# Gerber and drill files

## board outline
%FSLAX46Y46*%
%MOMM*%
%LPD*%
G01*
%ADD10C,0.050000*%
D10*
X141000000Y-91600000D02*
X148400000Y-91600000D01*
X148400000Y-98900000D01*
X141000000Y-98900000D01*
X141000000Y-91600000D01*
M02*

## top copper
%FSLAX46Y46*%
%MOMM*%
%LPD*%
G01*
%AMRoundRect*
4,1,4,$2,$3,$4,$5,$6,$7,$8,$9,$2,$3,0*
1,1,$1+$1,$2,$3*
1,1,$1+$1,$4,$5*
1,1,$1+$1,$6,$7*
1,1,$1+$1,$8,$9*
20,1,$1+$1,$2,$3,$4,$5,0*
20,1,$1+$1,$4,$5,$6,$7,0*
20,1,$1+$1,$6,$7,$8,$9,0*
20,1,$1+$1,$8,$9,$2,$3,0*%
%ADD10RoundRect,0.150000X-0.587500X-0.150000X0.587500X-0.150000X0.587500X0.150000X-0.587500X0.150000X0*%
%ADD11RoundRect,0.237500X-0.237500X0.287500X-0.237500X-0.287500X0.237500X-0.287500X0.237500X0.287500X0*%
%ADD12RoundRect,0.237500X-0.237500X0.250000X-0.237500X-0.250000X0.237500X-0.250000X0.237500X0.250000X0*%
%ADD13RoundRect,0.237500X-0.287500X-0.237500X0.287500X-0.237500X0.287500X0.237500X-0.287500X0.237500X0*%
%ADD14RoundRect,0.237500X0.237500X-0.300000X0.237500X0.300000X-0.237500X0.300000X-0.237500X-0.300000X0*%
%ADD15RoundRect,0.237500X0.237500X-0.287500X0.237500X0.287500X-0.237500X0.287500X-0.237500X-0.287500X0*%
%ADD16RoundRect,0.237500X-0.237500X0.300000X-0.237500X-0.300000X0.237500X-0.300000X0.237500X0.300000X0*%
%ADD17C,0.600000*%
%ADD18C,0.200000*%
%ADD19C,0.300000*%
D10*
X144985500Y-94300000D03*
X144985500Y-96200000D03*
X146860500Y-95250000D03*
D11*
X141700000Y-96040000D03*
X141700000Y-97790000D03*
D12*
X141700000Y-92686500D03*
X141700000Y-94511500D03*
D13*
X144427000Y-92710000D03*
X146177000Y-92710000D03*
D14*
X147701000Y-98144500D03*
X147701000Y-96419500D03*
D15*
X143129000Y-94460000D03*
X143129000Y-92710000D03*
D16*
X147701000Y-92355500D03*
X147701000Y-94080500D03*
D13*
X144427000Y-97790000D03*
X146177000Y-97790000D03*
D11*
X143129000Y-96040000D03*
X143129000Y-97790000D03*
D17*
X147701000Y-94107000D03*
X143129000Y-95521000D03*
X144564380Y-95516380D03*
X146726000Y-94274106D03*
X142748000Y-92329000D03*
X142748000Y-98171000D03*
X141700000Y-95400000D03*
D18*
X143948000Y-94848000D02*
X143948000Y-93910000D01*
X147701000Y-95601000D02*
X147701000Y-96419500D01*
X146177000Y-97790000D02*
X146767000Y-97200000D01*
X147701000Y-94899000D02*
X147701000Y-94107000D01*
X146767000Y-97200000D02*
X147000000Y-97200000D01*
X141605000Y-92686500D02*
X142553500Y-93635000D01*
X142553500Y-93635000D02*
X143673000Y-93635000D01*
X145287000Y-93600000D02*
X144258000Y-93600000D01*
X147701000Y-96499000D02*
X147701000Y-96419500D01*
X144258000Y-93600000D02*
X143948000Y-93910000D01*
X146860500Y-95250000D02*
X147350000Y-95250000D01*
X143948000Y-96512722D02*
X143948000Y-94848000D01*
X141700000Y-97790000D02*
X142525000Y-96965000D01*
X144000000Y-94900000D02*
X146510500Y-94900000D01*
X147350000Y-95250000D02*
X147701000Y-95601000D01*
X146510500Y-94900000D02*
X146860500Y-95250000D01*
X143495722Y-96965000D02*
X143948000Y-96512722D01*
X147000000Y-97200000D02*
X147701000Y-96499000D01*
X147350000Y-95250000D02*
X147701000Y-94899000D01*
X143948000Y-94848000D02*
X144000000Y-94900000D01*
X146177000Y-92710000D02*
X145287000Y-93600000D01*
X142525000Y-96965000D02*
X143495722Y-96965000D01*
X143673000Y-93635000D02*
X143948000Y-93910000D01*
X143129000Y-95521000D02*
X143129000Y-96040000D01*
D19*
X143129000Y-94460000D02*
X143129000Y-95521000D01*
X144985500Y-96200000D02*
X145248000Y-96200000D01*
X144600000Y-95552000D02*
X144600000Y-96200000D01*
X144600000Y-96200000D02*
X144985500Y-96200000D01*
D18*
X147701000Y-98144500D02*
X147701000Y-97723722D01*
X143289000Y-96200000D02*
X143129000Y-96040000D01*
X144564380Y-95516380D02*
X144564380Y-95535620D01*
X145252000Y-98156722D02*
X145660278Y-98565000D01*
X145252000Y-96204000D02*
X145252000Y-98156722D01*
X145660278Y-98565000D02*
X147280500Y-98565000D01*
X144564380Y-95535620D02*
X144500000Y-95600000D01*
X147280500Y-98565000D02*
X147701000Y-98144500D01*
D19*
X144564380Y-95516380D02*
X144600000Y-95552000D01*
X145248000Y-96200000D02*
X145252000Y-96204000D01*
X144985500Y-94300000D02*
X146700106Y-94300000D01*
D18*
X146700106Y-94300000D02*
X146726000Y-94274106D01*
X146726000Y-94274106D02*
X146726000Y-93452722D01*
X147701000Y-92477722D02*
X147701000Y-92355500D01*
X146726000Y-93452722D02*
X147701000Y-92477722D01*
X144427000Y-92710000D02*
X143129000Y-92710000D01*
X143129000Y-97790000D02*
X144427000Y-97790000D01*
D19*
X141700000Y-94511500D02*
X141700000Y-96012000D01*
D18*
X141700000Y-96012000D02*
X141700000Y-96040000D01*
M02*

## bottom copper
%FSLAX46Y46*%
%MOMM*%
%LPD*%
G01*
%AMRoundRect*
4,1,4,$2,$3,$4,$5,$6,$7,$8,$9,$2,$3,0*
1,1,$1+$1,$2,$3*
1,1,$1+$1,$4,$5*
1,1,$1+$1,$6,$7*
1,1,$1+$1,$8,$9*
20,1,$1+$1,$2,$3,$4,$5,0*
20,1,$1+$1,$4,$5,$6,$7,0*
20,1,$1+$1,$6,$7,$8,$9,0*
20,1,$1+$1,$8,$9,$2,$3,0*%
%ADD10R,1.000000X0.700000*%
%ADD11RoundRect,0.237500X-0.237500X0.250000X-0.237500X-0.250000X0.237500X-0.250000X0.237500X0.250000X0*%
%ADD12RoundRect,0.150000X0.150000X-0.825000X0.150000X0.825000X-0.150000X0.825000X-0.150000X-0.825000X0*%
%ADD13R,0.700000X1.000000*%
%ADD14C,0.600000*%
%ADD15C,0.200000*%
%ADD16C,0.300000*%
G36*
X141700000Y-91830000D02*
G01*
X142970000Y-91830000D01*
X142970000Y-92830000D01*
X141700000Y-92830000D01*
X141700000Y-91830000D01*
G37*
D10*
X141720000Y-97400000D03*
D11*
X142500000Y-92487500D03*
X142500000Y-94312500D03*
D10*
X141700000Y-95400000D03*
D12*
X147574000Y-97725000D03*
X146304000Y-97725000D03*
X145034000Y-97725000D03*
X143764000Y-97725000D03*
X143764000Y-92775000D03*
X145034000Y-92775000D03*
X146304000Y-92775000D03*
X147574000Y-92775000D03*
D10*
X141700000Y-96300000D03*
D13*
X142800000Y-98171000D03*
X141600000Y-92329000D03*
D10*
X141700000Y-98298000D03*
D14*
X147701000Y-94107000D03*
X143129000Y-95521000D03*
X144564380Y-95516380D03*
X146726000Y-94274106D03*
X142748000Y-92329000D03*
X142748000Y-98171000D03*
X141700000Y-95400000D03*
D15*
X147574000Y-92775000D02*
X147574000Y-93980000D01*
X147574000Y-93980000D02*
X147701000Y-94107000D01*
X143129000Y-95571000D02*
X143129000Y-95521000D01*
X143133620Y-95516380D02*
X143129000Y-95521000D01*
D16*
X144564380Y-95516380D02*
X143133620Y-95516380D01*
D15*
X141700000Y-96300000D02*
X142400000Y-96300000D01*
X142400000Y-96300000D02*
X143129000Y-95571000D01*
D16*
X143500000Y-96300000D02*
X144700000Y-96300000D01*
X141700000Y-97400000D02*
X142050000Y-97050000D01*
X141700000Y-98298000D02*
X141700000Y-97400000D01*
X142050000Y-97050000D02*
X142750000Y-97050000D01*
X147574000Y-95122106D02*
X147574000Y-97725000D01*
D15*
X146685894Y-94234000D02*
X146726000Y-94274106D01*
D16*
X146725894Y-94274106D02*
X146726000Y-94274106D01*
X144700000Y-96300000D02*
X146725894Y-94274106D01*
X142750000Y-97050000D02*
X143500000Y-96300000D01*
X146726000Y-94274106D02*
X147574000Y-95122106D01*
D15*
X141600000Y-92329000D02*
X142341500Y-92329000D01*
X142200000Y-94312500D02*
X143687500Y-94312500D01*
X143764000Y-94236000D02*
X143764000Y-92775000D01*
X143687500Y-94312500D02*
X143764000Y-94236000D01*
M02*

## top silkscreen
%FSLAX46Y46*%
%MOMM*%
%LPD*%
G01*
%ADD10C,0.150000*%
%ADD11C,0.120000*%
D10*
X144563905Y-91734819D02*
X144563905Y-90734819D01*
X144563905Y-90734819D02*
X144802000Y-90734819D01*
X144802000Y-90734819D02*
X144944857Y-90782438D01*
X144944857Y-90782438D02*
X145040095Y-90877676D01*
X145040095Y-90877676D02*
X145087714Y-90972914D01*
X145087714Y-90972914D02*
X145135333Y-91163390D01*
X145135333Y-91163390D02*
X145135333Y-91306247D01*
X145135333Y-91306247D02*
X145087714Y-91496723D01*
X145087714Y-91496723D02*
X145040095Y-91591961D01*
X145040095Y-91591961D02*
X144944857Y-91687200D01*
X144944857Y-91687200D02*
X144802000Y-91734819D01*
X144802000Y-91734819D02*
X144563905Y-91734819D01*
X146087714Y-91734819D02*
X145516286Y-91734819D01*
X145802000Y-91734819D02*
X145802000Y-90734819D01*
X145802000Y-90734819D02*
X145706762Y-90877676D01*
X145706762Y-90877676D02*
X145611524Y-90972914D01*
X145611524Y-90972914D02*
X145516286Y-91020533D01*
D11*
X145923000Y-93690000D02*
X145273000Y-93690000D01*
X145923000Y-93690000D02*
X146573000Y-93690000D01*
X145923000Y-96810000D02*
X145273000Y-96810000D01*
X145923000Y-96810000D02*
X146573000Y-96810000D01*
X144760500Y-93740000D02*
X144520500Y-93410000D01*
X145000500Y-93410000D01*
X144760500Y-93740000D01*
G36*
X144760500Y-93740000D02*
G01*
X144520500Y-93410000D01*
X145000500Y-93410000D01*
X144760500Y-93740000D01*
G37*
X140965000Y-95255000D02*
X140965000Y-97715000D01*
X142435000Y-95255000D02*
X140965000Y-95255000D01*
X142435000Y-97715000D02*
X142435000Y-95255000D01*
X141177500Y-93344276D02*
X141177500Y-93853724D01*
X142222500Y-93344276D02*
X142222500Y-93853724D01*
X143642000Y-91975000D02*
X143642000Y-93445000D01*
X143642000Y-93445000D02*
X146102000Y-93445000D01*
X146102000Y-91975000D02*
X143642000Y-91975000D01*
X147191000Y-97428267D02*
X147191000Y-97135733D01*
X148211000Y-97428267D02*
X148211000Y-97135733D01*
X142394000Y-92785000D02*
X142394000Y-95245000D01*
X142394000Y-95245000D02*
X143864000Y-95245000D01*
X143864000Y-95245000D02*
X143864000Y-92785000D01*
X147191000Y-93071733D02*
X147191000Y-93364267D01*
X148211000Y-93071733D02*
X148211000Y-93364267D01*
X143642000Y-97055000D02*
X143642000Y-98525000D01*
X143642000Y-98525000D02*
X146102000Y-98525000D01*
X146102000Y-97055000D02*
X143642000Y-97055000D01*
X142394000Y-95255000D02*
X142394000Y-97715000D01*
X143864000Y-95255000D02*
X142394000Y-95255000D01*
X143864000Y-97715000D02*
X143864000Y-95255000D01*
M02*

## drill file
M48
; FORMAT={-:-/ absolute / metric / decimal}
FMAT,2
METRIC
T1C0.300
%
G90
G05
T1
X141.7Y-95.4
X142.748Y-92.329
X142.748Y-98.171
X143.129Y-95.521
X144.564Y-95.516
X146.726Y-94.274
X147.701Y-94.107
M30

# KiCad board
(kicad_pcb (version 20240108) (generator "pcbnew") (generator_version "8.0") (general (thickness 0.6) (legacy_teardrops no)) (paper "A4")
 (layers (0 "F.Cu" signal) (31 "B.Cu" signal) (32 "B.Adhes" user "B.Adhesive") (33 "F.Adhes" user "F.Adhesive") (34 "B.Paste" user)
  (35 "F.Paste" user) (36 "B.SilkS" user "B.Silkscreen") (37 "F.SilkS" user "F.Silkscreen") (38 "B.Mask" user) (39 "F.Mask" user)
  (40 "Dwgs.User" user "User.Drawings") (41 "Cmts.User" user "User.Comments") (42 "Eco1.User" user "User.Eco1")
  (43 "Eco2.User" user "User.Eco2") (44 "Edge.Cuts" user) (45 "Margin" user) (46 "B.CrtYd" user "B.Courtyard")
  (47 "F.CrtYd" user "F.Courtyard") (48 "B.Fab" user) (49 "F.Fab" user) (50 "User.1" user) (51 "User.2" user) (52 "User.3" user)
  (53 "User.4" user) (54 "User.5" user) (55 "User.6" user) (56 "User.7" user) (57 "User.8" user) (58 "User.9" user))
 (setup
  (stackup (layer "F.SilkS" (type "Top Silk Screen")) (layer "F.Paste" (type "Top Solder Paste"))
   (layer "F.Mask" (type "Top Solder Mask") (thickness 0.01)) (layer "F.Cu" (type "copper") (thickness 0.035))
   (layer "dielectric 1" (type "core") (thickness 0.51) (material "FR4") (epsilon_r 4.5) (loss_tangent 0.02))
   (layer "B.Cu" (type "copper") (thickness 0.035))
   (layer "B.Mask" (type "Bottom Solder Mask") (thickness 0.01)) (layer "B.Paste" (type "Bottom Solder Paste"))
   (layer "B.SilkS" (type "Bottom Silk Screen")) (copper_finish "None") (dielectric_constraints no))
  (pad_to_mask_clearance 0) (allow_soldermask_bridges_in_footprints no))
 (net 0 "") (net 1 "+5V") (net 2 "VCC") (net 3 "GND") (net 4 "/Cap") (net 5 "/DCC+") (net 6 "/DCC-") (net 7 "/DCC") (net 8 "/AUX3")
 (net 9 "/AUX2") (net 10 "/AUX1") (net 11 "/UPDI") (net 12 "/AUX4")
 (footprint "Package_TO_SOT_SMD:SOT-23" (layer "F.Cu") (at 145.923 95.25)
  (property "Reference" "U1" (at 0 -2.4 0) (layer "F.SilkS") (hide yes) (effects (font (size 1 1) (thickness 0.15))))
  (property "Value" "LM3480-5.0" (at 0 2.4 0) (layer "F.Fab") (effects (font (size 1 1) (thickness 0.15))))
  (fp_line (start 0 -1.56) (end -0.65 -1.56) (stroke (width 0.12) (type solid)) (layer "F.SilkS"))
  (fp_line (start 0 -1.56) (end 0.65 -1.56) (stroke (width 0.12) (type solid)) (layer "F.SilkS"))
  (fp_line (start 0 1.56) (end -0.65 1.56) (stroke (width 0.12) (type solid)) (layer "F.SilkS"))
  (fp_line (start 0 1.56) (end 0.65 1.56) (stroke (width 0.12) (type solid)) (layer "F.SilkS"))
  (fp_poly
   (pts (xy -1.1625 -1.51) (xy -1.4025 -1.84) (xy -0.9225 -1.84) (xy -1.1625 -1.51)) (stroke (width 0.12) (type solid)) (fill solid)
   (layer "F.SilkS"))
  (pad "1" smd roundrect (at -0.9375 -0.95) (size 1.475 0.6) (layers "F.Cu" "F.Paste" "F.Mask") (roundrect_rratio 0.25) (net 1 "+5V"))
  (pad "2" smd roundrect (at -0.9375 0.95) (size 1.475 0.6) (layers "F.Cu" "F.Paste" "F.Mask") (roundrect_rratio 0.25) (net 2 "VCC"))
  (pad "3" smd roundrect (at 0.9375 0) (size 1.475 0.6) (layers "F.Cu" "F.Paste" "F.Mask") (roundrect_rratio 0.25) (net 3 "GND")))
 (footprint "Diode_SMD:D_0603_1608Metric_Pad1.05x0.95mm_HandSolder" (layer "F.Cu") (at 141.7 96.915 -90)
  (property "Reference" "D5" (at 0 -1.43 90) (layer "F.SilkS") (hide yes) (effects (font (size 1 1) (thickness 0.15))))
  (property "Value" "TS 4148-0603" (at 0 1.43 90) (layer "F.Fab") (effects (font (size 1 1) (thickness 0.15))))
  (fp_line (start -1.66 0.735) (end 0.8 0.735) (stroke (width 0.12) (type solid)) (layer "F.SilkS"))
  (fp_line (start -1.66 -0.735) (end -1.66 0.735) (stroke (width 0.12) (type solid)) (layer "F.SilkS"))
  (fp_line (start 0.8 -0.735) (end -1.66 -0.735) (stroke (width 0.12) (type solid)) (layer "F.SilkS"))
  (pad "1" smd roundrect (at -0.875 0 270) (size 1.05 0.95) (layers "F.Cu" "F.Paste" "F.Mask") (roundrect_rratio 0.25) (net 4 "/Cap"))
  (pad "2" smd roundrect (at 0.875 0 270) (size 1.05 0.95) (layers "F.Cu" "F.Paste" "F.Mask") (roundrect_rratio 0.25) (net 3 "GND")))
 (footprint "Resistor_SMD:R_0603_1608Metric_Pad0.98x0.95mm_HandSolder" (layer "F.Cu") (at 141.7 93.599 -90)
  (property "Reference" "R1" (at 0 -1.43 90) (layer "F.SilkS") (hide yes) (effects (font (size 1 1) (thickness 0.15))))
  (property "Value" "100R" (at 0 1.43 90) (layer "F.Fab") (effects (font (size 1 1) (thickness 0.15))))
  (fp_line (start -0.254724 0.5225) (end 0.254724 0.5225) (stroke (width 0.12) (type solid)) (layer "F.SilkS"))
  (fp_line (start -0.254724 -0.5225) (end 0.254724 -0.5225) (stroke (width 0.12) (type solid)) (layer "F.SilkS"))
  (pad "1" smd roundrect (at -0.9125 0 270) (size 0.975 0.95) (layers "F.Cu" "F.Paste" "F.Mask") (roundrect_rratio 0.25) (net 3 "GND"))
  (pad "2" smd roundrect (at 0.9125 0 270) (size 0.975 0.95) (layers "F.Cu" "F.Paste" "F.Mask") (roundrect_rratio 0.25) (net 4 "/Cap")))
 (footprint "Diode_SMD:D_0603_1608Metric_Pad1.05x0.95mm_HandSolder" (layer "F.Cu") (at 145.302 92.71)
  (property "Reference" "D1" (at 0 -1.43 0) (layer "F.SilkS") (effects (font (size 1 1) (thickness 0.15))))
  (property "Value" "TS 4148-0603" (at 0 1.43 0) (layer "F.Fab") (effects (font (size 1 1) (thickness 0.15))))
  (fp_line (start -1.66 -0.735) (end -1.66 0.735) (stroke (width 0.12) (type solid)) (layer "F.SilkS"))
  (fp_line (start -1.66 0.735) (end 0.8 0.735) (stroke (width 0.12) (type solid)) (layer "F.SilkS"))
  (fp_line (start 0.8 -0.735) (end -1.66 -0.735) (stroke (width 0.12) (type solid)) (layer "F.SilkS"))
  (pad "1" smd roundrect (at -0.875 0) (size 1.05 0.95) (layers "F.Cu" "F.Paste" "F.Mask") (roundrect_rratio 0.25) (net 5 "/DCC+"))
  (pad "2" smd roundrect (at 0.875 0) (size 1.05 0.95) (layers "F.Cu" "F.Paste" "F.Mask") (roundrect_rratio 0.25) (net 3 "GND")))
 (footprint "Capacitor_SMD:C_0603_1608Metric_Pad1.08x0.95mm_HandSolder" (layer "F.Cu") (at 147.701 97.282 90)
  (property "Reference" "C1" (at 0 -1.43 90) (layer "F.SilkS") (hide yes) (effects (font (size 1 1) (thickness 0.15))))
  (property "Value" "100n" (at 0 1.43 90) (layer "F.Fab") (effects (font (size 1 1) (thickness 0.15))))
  (fp_line (start -0.146267 -0.51) (end 0.146267 -0.51) (stroke (width 0.12) (type solid)) (layer "F.SilkS"))
  (fp_line (start -0.146267 0.51) (end 0.146267 0.51) (stroke (width 0.12) (type solid)) (layer "F.SilkS"))
  (pad "1" smd roundrect (at -0.8625 0 90) (size 1.075 0.95) (layers "F.Cu" "F.Paste" "F.Mask") (roundrect_rratio 0.25) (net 2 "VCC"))
  (pad "2" smd roundrect (at 0.8625 0 90) (size 1.075 0.95) (layers "F.Cu" "F.Paste" "F.Mask") (roundrect_rratio 0.25) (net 3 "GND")))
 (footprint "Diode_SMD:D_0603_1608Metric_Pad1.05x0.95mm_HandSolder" (layer "F.Cu") (at 143.129 93.585 90)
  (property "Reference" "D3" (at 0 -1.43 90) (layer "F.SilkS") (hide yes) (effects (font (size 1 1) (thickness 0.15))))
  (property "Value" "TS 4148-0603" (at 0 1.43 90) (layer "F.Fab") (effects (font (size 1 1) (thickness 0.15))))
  (fp_line (start 0.8 -0.735) (end -1.66 -0.735) (stroke (width 0.12) (type solid)) (layer "F.SilkS"))
  (fp_line (start -1.66 -0.735) (end -1.66 0.735) (stroke (width 0.12) (type solid)) (layer "F.SilkS"))
  (fp_line (start -1.66 0.735) (end 0.8 0.735) (stroke (width 0.12) (type solid)) (layer "F.SilkS"))
  (pad "1" smd roundrect (at -0.875 0 90) (size 1.05 0.95) (layers "F.Cu" "F.Paste" "F.Mask") (roundrect_rratio 0.25) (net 2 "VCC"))
  (pad "2" smd roundrect (at 0.875 0 90) (size 1.05 0.95) (layers "F.Cu" "F.Paste" "F.Mask") (roundrect_rratio 0.25) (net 5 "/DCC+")))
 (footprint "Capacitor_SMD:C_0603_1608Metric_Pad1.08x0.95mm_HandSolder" (layer "F.Cu") (at 147.701 93.218 -90)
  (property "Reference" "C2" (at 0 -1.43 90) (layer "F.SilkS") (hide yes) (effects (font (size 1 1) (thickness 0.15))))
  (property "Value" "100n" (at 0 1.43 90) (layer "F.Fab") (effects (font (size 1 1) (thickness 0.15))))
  (fp_line (start -0.146267 0.51) (end 0.146267 0.51) (stroke (width 0.12) (type solid)) (layer "F.SilkS"))
  (fp_line (start -0.146267 -0.51) (end 0.146267 -0.51) (stroke (width 0.12) (type solid)) (layer "F.SilkS"))
  (pad "1" smd roundrect (at -0.8625 0 270) (size 1.075 0.95) (layers "F.Cu" "F.Paste" "F.Mask") (roundrect_rratio 0.25) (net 1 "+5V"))
  (pad "2" smd roundrect (at 0.8625 0 270) (size 1.075 0.95) (layers "F.Cu" "F.Paste" "F.Mask") (roundrect_rratio 0.25) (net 3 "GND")))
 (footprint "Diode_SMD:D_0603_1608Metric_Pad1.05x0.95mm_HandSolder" (layer "F.Cu") (at 145.302 97.79)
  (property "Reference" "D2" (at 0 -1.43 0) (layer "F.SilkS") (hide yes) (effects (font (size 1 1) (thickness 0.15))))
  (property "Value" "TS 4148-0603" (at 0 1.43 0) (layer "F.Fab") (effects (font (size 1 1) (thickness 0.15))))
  (fp_line (start -1.66 -0.735) (end -1.66 0.735) (stroke (width 0.12) (type solid)) (layer "F.SilkS"))
  (fp_line (start -1.66 0.735) (end 0.8 0.735) (stroke (width 0.12) (type solid)) (layer "F.SilkS"))
  (fp_line (start 0.8 -0.735) (end -1.66 -0.735) (stroke (width 0.12) (type solid)) (layer "F.SilkS"))
  (pad "1" smd roundrect (at -0.875 0) (size 1.05 0.95) (layers "F.Cu" "F.Paste" "F.Mask") (roundrect_rratio 0.25) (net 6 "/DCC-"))
  (pad "2" smd roundrect (at 0.875 0) (size 1.05 0.95) (layers "F.Cu" "F.Paste" "F.Mask") (roundrect_rratio 0.25) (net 3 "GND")))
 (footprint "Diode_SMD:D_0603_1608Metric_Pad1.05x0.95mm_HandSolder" (layer "F.Cu") (at 143.129 96.915 -90)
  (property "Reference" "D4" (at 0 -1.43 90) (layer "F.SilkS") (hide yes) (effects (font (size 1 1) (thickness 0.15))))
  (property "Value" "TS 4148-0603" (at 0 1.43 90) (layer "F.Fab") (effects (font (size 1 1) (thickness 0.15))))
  (fp_line (start -1.66 0.735) (end 0.8 0.735) (stroke (width 0.12) (type solid)) (layer "F.SilkS"))
  (fp_line (start -1.66 -0.735) (end -1.66 0.735) (stroke (width 0.12) (type solid)) (layer "F.SilkS"))
  (fp_line (start 0.8 -0.735) (end -1.66 -0.735) (stroke (width 0.12) (type solid)) (layer "F.SilkS"))
  (pad "1" smd roundrect (at -0.875 0 270) (size 1.05 0.95) (layers "F.Cu" "F.Paste" "F.Mask") (roundrect_rratio 0.25) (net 2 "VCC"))
  (pad "2" smd roundrect (at 0.875 0 270) (size 1.05 0.95) (layers "F.Cu" "F.Paste" "F.Mask") (roundrect_rratio 0.25) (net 6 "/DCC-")))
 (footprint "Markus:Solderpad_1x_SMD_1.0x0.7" (layer "B.Cu") (at 141.72 97.4 180)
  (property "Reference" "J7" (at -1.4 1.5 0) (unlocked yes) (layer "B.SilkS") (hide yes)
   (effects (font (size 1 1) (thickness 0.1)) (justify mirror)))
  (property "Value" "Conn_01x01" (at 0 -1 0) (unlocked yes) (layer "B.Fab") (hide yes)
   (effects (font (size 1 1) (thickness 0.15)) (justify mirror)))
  (pad "1" smd rect (at 0 0 180) (size 1 0.7) (layers "B.Cu" "B.Paste" "B.Mask") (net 1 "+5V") (thermal_bridge_angle 45)))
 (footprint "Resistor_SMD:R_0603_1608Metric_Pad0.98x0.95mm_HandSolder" (layer "B.Cu") (at 142.5 93.4 -90)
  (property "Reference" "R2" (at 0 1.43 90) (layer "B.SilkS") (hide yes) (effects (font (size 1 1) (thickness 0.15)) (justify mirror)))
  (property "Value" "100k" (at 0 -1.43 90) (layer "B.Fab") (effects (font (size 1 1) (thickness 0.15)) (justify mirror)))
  (pad "1" smd roundrect (at -0.9125 0 270) (size 0.975 0.95) (layers "B.Cu" "B.Paste" "B.Mask") (roundrect_rratio 0.25) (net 5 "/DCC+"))
  (pad "2" smd roundrect (at 0.9125 0 270) (size 0.975 0.95) (layers "B.Cu" "B.Paste" "B.Mask") (roundrect_rratio 0.25) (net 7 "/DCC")))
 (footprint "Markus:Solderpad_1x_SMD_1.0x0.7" (layer "B.Cu") (at 141.7 95.4 180)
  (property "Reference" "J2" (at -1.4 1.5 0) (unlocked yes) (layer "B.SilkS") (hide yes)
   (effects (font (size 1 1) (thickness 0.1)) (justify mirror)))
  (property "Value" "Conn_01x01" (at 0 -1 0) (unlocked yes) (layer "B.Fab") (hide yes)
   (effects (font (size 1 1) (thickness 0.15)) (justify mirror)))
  (pad "1" smd rect (at 0 0 180) (size 1 0.7) (layers "B.Cu" "B.Paste" "B.Mask") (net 4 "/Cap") (thermal_bridge_angle 45)))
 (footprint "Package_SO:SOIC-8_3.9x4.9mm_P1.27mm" (layer "B.Cu") (at 145.669 95.25 90)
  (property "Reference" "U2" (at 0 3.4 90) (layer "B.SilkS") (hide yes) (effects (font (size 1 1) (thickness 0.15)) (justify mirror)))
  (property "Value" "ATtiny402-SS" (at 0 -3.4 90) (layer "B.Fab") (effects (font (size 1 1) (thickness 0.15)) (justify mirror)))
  (pad "1" smd roundrect (at -2.475 1.905 90) (size 1.95 0.6) (layers "B.Cu" "B.Paste" "B.Mask") (roundrect_rratio 0.25) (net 1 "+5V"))
  (pad "2" smd roundrect (at -2.475 0.635 90) (size 1.95 0.6) (layers "B.Cu" "B.Paste" "B.Mask") (roundrect_rratio 0.25) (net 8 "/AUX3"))
  (pad "3" smd roundrect (at -2.475 -0.635 90) (size 1.95 0.6) (layers "B.Cu" "B.Paste" "B.Mask") (roundrect_rratio 0.25) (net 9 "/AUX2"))
  (pad "4" smd roundrect (at -2.475 -1.905 90) (size 1.95 0.6) (layers "B.Cu" "B.Paste" "B.Mask") (roundrect_rratio 0.25) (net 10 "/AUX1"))
  (pad "5" smd roundrect (at 2.475 -1.905 90) (size 1.95 0.6) (layers "B.Cu" "B.Paste" "B.Mask") (roundrect_rratio 0.25) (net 7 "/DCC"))
  (pad "6" smd roundrect (at 2.475 -0.635 90) (size 1.95 0.6) (layers "B.Cu" "B.Paste" "B.Mask") (roundrect_rratio 0.25) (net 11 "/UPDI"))
  (pad "7" smd roundrect (at 2.475 0.635 90) (size 1.95 0.6) (layers "B.Cu" "B.Paste" "B.Mask") (roundrect_rratio 0.25) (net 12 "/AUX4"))
  (pad "8" smd roundrect (at 2.475 1.905 90) (size 1.95 0.6) (layers "B.Cu" "B.Paste" "B.Mask") (roundrect_rratio 0.25) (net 3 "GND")))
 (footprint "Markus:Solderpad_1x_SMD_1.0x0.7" (layer "B.Cu") (at 141.7 96.3 180)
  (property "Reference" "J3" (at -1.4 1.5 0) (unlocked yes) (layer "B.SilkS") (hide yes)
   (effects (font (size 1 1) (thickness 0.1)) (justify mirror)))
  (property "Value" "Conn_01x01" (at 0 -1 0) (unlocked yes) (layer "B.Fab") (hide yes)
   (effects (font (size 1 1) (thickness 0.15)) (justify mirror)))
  (pad "1" smd rect (at 0 0 180) (size 1 0.7) (layers "B.Cu" "B.Paste" "B.Mask") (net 2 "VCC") (thermal_bridge_angle 45)))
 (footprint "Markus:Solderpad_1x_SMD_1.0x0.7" (layer "B.Cu") (at 142.8 98.171 -90)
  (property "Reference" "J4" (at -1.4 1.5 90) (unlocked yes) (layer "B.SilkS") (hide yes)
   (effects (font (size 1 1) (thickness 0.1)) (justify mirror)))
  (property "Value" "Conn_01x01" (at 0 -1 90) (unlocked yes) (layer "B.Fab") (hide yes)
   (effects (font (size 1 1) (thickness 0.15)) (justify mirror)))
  (pad "1" smd rect (at 0 0 270) (size 1 0.7) (layers "B.Cu" "B.Paste" "B.Mask") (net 6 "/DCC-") (thermal_bridge_angle 45)))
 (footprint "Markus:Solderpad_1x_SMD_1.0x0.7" (layer "B.Cu") (at 141.6 92.329 -90)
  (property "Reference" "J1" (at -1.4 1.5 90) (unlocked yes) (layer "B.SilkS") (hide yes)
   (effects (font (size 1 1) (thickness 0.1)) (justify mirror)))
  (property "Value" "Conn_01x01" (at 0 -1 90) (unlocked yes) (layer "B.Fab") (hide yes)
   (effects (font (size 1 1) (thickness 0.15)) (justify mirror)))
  (pad "1" smd rect (at 0 0 270) (size 1 0.7) (layers "B.Cu" "B.Paste" "B.Mask") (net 5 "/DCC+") (thermal_bridge_angle 45)))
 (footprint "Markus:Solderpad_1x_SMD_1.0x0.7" (layer "B.Cu") (at 141.7 98.298 180)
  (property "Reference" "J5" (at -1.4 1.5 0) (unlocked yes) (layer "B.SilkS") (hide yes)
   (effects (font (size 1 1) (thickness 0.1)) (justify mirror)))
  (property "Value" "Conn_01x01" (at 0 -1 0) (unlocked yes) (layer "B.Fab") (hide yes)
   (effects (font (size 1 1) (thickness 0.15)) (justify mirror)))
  (pad "1" smd rect (at 0 0 180) (size 1 0.7) (layers "B.Cu" "B.Paste" "B.Mask") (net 1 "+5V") (thermal_bridge_angle 45)))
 (gr_rect (start 141.7 91.83) (end 142.97 92.83) (stroke (width 0) (type solid)) (fill solid) (layer "B.Cu") (net 5))
 (gr_rect (start 141 91.6) (end 148.4 98.9) (stroke (width 0.05) (type default)) (fill none) (layer "Edge.Cuts"))
 (segment (start 143.948 94.848) (end 143.948 93.91) (width 0.2) (layer "F.Cu") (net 3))
 (segment (start 147.701 95.601) (end 147.701 96.4195) (width 0.2) (layer "F.Cu") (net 3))
 (segment (start 146.177 97.79) (end 146.767 97.2) (width 0.2) (layer "F.Cu") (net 3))
 (segment (start 147.701 94.899) (end 147.701 94.107) (width 0.2) (layer "F.Cu") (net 3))
 (segment (start 146.767 97.2) (end 147 97.2) (width 0.2) (layer "F.Cu") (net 3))
 (segment (start 141.605 92.6865) (end 142.5535 93.635) (width 0.2) (layer "F.Cu") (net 3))
 (segment (start 142.5535 93.635) (end 143.673 93.635) (width 0.2) (layer "F.Cu") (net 3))
 (segment (start 145.287 93.6) (end 144.258 93.6) (width 0.2) (layer "F.Cu") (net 3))
 (segment (start 147.701 96.499) (end 147.701 96.4195) (width 0.2) (layer "F.Cu") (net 3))
 (segment (start 144.258 93.6) (end 143.948 93.91) (width 0.2) (layer "F.Cu") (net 3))
 (segment (start 146.8605 95.25) (end 147.35 95.25) (width 0.2) (layer "F.Cu") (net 3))
 (segment (start 143.948 96.512722) (end 143.948 94.848) (width 0.2) (layer "F.Cu") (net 3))
 (segment (start 141.7 97.79) (end 142.525 96.965) (width 0.2) (layer "F.Cu") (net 3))
 (segment (start 144 94.9) (end 146.5105 94.9) (width 0.2) (layer "F.Cu") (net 3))
 (segment (start 147.35 95.25) (end 147.701 95.601) (width 0.2) (layer "F.Cu") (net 3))
 (segment (start 146.5105 94.9) (end 146.8605 95.25) (width 0.2) (layer "F.Cu") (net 3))
 (segment (start 143.495722 96.965) (end 143.948 96.512722) (width 0.2) (layer "F.Cu") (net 3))
 (segment (start 147 97.2) (end 147.701 96.499) (width 0.2) (layer "F.Cu") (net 3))
 (segment (start 147.35 95.25) (end 147.701 94.899) (width 0.2) (layer "F.Cu") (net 3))
 (segment (start 143.948 94.848) (end 144 94.9) (width 0.2) (layer "F.Cu") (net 3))
 (segment (start 146.177 92.71) (end 145.287 93.6) (width 0.2) (layer "F.Cu") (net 3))
 (segment (start 142.525 96.965) (end 143.495722 96.965) (width 0.2) (layer "F.Cu") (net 3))
 (segment (start 143.673 93.635) (end 143.948 93.91) (width 0.2) (layer "F.Cu") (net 3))
 (via (at 147.701 94.107) (size 0.6) (drill 0.3) (layers "F.Cu" "B.Cu") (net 3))
 (segment (start 147.574 92.775) (end 147.574 93.98) (width 0.2) (layer "B.Cu") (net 3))
 (segment (start 147.574 93.98) (end 147.701 94.107) (width 0.2) (layer "B.Cu") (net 3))
 (segment (start 143.129 95.521) (end 143.129 96.04) (width 0.2) (layer "F.Cu") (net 2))
 (segment (start 143.129 94.46) (end 143.129 95.521) (width 0.3) (layer "F.Cu") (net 2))
 (segment (start 144.9855 96.2) (end 145.248 96.2) (width 0.3) (layer "F.Cu") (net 2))
 (segment (start 144.6 95.552) (end 144.6 96.2) (width 0.3) (layer "F.Cu") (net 2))
 (segment (start 144.6 96.2) (end 144.9855 96.2) (width 0.3) (layer "F.Cu") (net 2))
 (segment (start 147.701 98.1445) (end 147.701 97.723722) (width 0.2) (layer "F.Cu") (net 2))
 (segment (start 143.289 96.2) (end 143.129 96.04) (width 0.2) (layer "F.Cu") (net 2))
 (segment (start 144.56438 95.51638) (end 144.56438 95.53562) (width 0.2) (layer "F.Cu") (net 2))
 (segment (start 145.252 98.156722) (end 145.660278 98.565) (width 0.2) (layer "F.Cu") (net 2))
 (segment (start 145.252 96.204) (end 145.252 98.156722) (width 0.2) (layer "F.Cu") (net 2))
 (segment (start 145.660278 98.565) (end 147.2805 98.565) (width 0.2) (layer "F.Cu") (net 2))
 (segment (start 144.56438 95.53562) (end 144.5 95.6) (width 0.2) (layer "F.Cu") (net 2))
 (segment (start 147.2805 98.565) (end 147.701 98.1445) (width 0.2) (layer "F.Cu") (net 2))
 (segment (start 144.56438 95.51638) (end 144.6 95.552) (width 0.3) (layer "F.Cu") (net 2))
 (segment (start 145.248 96.2) (end 145.252 96.204) (width 0.3) (layer "F.Cu") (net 2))
 (via (at 143.129 95.521) (size 0.6) (drill 0.3) (layers "F.Cu" "B.Cu") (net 2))
 (via (at 144.56438 95.51638) (size 0.6) (drill 0.3) (layers "F.Cu" "B.Cu") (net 2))
 (segment (start 143.129 95.571) (end 143.129 95.521) (width 0.2) (layer "B.Cu") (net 2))
 (segment (start 143.13362 95.51638) (end 143.129 95.521) (width 0.2) (layer "B.Cu") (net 2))
 (segment (start 144.56438 95.51638) (end 143.13362 95.51638) (width 0.3) (layer "B.Cu") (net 2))
 (segment (start 141.7 96.3) (end 142.4 96.3) (width 0.2) (layer "B.Cu") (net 2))
 (segment (start 142.4 96.3) (end 143.129 95.571) (width 0.2) (layer "B.Cu") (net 2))
 (segment (start 144.9855 94.3) (end 146.700106 94.3) (width 0.3) (layer "F.Cu") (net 1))
 (segment (start 146.700106 94.3) (end 146.726 94.274106) (width 0.2) (layer "F.Cu") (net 1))
 (segment (start 146.726 94.274106) (end 146.726 93.452722) (width 0.2) (layer "F.Cu") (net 1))
 (segment (start 147.701 92.477722) (end 147.701 92.3555) (width 0.2) (layer "F.Cu") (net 1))
 (segment (start 146.726 93.452722) (end 147.701 92.477722) (width 0.2) (layer "F.Cu") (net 1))
 (via (at 146.726 94.274106) (size 0.6) (drill 0.3) (layers "F.Cu" "B.Cu") (free yes) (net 1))
 (segment (start 143.5 96.3) (end 144.7 96.3) (width 0.3) (layer "B.Cu") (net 1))
 (segment (start 141.7 97.4) (end 142.05 97.05) (width 0.3) (layer "B.Cu") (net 1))
 (segment (start 141.7 98.298) (end 141.7 97.4) (width 0.3) (layer "B.Cu") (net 1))
 (segment (start 142.05 97.05) (end 142.75 97.05) (width 0.3) (layer "B.Cu") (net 1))
 (segment (start 147.574 95.122106) (end 147.574 97.725) (width 0.3) (layer "B.Cu") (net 1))
 (segment (start 146.685894 94.234) (end 146.726 94.274106) (width 0.2) (layer "B.Cu") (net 1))
 (segment (start 146.725894 94.274106) (end 146.726 94.274106) (width 0.3) (layer "B.Cu") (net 1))
 (segment (start 144.7 96.3) (end 146.725894 94.274106) (width 0.3) (layer "B.Cu") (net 1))
 (segment (start 142.75 97.05) (end 143.5 96.3) (width 0.3) (layer "B.Cu") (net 1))
 (segment (start 146.726 94.274106) (end 147.574 95.122106) (width 0.3) (layer "B.Cu") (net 1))
 (segment (start 144.427 92.71) (end 143.129 92.71) (width 0.2) (layer "F.Cu") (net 5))
 (via (at 142.748 92.329) (size 0.6) (drill 0.3) (layers "F.Cu" "B.Cu") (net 5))
 (segment (start 141.6 92.329) (end 142.3415 92.329) (width 0.2) (layer "B.Cu") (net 5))
 (segment (start 143.129 97.79) (end 144.427 97.79) (width 0.2) (layer "F.Cu") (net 6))
 (via (at 142.748 98.171) (size 0.6) (drill 0.3) (layers "F.Cu" "B.Cu") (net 6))
 (segment (start 141.7 94.5115) (end 141.7 96.012) (width 0.3) (layer "F.Cu") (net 4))
 (segment (start 141.7 96.012) (end 141.7 96.04) (width 0.2) (layer "F.Cu") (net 4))
 (via (at 141.7 95.4) (size 0.6) (drill 0.3) (layers "F.Cu" "B.Cu") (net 4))
 (segment (start 142.2 94.3125) (end 143.6875 94.3125) (width 0.2) (layer "B.Cu") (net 7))
 (segment (start 143.764 94.236) (end 143.764 92.775) (width 0.2) (layer "B.Cu") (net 7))
 (segment (start 143.6875 94.3125) (end 143.764 94.236) (width 0.2) (layer "B.Cu") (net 7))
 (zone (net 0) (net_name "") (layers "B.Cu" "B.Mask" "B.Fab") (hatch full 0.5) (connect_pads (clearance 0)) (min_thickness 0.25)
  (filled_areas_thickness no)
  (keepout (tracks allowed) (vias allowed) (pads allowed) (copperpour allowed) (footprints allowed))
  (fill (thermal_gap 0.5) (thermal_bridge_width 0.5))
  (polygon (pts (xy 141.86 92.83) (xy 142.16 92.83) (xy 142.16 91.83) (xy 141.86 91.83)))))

